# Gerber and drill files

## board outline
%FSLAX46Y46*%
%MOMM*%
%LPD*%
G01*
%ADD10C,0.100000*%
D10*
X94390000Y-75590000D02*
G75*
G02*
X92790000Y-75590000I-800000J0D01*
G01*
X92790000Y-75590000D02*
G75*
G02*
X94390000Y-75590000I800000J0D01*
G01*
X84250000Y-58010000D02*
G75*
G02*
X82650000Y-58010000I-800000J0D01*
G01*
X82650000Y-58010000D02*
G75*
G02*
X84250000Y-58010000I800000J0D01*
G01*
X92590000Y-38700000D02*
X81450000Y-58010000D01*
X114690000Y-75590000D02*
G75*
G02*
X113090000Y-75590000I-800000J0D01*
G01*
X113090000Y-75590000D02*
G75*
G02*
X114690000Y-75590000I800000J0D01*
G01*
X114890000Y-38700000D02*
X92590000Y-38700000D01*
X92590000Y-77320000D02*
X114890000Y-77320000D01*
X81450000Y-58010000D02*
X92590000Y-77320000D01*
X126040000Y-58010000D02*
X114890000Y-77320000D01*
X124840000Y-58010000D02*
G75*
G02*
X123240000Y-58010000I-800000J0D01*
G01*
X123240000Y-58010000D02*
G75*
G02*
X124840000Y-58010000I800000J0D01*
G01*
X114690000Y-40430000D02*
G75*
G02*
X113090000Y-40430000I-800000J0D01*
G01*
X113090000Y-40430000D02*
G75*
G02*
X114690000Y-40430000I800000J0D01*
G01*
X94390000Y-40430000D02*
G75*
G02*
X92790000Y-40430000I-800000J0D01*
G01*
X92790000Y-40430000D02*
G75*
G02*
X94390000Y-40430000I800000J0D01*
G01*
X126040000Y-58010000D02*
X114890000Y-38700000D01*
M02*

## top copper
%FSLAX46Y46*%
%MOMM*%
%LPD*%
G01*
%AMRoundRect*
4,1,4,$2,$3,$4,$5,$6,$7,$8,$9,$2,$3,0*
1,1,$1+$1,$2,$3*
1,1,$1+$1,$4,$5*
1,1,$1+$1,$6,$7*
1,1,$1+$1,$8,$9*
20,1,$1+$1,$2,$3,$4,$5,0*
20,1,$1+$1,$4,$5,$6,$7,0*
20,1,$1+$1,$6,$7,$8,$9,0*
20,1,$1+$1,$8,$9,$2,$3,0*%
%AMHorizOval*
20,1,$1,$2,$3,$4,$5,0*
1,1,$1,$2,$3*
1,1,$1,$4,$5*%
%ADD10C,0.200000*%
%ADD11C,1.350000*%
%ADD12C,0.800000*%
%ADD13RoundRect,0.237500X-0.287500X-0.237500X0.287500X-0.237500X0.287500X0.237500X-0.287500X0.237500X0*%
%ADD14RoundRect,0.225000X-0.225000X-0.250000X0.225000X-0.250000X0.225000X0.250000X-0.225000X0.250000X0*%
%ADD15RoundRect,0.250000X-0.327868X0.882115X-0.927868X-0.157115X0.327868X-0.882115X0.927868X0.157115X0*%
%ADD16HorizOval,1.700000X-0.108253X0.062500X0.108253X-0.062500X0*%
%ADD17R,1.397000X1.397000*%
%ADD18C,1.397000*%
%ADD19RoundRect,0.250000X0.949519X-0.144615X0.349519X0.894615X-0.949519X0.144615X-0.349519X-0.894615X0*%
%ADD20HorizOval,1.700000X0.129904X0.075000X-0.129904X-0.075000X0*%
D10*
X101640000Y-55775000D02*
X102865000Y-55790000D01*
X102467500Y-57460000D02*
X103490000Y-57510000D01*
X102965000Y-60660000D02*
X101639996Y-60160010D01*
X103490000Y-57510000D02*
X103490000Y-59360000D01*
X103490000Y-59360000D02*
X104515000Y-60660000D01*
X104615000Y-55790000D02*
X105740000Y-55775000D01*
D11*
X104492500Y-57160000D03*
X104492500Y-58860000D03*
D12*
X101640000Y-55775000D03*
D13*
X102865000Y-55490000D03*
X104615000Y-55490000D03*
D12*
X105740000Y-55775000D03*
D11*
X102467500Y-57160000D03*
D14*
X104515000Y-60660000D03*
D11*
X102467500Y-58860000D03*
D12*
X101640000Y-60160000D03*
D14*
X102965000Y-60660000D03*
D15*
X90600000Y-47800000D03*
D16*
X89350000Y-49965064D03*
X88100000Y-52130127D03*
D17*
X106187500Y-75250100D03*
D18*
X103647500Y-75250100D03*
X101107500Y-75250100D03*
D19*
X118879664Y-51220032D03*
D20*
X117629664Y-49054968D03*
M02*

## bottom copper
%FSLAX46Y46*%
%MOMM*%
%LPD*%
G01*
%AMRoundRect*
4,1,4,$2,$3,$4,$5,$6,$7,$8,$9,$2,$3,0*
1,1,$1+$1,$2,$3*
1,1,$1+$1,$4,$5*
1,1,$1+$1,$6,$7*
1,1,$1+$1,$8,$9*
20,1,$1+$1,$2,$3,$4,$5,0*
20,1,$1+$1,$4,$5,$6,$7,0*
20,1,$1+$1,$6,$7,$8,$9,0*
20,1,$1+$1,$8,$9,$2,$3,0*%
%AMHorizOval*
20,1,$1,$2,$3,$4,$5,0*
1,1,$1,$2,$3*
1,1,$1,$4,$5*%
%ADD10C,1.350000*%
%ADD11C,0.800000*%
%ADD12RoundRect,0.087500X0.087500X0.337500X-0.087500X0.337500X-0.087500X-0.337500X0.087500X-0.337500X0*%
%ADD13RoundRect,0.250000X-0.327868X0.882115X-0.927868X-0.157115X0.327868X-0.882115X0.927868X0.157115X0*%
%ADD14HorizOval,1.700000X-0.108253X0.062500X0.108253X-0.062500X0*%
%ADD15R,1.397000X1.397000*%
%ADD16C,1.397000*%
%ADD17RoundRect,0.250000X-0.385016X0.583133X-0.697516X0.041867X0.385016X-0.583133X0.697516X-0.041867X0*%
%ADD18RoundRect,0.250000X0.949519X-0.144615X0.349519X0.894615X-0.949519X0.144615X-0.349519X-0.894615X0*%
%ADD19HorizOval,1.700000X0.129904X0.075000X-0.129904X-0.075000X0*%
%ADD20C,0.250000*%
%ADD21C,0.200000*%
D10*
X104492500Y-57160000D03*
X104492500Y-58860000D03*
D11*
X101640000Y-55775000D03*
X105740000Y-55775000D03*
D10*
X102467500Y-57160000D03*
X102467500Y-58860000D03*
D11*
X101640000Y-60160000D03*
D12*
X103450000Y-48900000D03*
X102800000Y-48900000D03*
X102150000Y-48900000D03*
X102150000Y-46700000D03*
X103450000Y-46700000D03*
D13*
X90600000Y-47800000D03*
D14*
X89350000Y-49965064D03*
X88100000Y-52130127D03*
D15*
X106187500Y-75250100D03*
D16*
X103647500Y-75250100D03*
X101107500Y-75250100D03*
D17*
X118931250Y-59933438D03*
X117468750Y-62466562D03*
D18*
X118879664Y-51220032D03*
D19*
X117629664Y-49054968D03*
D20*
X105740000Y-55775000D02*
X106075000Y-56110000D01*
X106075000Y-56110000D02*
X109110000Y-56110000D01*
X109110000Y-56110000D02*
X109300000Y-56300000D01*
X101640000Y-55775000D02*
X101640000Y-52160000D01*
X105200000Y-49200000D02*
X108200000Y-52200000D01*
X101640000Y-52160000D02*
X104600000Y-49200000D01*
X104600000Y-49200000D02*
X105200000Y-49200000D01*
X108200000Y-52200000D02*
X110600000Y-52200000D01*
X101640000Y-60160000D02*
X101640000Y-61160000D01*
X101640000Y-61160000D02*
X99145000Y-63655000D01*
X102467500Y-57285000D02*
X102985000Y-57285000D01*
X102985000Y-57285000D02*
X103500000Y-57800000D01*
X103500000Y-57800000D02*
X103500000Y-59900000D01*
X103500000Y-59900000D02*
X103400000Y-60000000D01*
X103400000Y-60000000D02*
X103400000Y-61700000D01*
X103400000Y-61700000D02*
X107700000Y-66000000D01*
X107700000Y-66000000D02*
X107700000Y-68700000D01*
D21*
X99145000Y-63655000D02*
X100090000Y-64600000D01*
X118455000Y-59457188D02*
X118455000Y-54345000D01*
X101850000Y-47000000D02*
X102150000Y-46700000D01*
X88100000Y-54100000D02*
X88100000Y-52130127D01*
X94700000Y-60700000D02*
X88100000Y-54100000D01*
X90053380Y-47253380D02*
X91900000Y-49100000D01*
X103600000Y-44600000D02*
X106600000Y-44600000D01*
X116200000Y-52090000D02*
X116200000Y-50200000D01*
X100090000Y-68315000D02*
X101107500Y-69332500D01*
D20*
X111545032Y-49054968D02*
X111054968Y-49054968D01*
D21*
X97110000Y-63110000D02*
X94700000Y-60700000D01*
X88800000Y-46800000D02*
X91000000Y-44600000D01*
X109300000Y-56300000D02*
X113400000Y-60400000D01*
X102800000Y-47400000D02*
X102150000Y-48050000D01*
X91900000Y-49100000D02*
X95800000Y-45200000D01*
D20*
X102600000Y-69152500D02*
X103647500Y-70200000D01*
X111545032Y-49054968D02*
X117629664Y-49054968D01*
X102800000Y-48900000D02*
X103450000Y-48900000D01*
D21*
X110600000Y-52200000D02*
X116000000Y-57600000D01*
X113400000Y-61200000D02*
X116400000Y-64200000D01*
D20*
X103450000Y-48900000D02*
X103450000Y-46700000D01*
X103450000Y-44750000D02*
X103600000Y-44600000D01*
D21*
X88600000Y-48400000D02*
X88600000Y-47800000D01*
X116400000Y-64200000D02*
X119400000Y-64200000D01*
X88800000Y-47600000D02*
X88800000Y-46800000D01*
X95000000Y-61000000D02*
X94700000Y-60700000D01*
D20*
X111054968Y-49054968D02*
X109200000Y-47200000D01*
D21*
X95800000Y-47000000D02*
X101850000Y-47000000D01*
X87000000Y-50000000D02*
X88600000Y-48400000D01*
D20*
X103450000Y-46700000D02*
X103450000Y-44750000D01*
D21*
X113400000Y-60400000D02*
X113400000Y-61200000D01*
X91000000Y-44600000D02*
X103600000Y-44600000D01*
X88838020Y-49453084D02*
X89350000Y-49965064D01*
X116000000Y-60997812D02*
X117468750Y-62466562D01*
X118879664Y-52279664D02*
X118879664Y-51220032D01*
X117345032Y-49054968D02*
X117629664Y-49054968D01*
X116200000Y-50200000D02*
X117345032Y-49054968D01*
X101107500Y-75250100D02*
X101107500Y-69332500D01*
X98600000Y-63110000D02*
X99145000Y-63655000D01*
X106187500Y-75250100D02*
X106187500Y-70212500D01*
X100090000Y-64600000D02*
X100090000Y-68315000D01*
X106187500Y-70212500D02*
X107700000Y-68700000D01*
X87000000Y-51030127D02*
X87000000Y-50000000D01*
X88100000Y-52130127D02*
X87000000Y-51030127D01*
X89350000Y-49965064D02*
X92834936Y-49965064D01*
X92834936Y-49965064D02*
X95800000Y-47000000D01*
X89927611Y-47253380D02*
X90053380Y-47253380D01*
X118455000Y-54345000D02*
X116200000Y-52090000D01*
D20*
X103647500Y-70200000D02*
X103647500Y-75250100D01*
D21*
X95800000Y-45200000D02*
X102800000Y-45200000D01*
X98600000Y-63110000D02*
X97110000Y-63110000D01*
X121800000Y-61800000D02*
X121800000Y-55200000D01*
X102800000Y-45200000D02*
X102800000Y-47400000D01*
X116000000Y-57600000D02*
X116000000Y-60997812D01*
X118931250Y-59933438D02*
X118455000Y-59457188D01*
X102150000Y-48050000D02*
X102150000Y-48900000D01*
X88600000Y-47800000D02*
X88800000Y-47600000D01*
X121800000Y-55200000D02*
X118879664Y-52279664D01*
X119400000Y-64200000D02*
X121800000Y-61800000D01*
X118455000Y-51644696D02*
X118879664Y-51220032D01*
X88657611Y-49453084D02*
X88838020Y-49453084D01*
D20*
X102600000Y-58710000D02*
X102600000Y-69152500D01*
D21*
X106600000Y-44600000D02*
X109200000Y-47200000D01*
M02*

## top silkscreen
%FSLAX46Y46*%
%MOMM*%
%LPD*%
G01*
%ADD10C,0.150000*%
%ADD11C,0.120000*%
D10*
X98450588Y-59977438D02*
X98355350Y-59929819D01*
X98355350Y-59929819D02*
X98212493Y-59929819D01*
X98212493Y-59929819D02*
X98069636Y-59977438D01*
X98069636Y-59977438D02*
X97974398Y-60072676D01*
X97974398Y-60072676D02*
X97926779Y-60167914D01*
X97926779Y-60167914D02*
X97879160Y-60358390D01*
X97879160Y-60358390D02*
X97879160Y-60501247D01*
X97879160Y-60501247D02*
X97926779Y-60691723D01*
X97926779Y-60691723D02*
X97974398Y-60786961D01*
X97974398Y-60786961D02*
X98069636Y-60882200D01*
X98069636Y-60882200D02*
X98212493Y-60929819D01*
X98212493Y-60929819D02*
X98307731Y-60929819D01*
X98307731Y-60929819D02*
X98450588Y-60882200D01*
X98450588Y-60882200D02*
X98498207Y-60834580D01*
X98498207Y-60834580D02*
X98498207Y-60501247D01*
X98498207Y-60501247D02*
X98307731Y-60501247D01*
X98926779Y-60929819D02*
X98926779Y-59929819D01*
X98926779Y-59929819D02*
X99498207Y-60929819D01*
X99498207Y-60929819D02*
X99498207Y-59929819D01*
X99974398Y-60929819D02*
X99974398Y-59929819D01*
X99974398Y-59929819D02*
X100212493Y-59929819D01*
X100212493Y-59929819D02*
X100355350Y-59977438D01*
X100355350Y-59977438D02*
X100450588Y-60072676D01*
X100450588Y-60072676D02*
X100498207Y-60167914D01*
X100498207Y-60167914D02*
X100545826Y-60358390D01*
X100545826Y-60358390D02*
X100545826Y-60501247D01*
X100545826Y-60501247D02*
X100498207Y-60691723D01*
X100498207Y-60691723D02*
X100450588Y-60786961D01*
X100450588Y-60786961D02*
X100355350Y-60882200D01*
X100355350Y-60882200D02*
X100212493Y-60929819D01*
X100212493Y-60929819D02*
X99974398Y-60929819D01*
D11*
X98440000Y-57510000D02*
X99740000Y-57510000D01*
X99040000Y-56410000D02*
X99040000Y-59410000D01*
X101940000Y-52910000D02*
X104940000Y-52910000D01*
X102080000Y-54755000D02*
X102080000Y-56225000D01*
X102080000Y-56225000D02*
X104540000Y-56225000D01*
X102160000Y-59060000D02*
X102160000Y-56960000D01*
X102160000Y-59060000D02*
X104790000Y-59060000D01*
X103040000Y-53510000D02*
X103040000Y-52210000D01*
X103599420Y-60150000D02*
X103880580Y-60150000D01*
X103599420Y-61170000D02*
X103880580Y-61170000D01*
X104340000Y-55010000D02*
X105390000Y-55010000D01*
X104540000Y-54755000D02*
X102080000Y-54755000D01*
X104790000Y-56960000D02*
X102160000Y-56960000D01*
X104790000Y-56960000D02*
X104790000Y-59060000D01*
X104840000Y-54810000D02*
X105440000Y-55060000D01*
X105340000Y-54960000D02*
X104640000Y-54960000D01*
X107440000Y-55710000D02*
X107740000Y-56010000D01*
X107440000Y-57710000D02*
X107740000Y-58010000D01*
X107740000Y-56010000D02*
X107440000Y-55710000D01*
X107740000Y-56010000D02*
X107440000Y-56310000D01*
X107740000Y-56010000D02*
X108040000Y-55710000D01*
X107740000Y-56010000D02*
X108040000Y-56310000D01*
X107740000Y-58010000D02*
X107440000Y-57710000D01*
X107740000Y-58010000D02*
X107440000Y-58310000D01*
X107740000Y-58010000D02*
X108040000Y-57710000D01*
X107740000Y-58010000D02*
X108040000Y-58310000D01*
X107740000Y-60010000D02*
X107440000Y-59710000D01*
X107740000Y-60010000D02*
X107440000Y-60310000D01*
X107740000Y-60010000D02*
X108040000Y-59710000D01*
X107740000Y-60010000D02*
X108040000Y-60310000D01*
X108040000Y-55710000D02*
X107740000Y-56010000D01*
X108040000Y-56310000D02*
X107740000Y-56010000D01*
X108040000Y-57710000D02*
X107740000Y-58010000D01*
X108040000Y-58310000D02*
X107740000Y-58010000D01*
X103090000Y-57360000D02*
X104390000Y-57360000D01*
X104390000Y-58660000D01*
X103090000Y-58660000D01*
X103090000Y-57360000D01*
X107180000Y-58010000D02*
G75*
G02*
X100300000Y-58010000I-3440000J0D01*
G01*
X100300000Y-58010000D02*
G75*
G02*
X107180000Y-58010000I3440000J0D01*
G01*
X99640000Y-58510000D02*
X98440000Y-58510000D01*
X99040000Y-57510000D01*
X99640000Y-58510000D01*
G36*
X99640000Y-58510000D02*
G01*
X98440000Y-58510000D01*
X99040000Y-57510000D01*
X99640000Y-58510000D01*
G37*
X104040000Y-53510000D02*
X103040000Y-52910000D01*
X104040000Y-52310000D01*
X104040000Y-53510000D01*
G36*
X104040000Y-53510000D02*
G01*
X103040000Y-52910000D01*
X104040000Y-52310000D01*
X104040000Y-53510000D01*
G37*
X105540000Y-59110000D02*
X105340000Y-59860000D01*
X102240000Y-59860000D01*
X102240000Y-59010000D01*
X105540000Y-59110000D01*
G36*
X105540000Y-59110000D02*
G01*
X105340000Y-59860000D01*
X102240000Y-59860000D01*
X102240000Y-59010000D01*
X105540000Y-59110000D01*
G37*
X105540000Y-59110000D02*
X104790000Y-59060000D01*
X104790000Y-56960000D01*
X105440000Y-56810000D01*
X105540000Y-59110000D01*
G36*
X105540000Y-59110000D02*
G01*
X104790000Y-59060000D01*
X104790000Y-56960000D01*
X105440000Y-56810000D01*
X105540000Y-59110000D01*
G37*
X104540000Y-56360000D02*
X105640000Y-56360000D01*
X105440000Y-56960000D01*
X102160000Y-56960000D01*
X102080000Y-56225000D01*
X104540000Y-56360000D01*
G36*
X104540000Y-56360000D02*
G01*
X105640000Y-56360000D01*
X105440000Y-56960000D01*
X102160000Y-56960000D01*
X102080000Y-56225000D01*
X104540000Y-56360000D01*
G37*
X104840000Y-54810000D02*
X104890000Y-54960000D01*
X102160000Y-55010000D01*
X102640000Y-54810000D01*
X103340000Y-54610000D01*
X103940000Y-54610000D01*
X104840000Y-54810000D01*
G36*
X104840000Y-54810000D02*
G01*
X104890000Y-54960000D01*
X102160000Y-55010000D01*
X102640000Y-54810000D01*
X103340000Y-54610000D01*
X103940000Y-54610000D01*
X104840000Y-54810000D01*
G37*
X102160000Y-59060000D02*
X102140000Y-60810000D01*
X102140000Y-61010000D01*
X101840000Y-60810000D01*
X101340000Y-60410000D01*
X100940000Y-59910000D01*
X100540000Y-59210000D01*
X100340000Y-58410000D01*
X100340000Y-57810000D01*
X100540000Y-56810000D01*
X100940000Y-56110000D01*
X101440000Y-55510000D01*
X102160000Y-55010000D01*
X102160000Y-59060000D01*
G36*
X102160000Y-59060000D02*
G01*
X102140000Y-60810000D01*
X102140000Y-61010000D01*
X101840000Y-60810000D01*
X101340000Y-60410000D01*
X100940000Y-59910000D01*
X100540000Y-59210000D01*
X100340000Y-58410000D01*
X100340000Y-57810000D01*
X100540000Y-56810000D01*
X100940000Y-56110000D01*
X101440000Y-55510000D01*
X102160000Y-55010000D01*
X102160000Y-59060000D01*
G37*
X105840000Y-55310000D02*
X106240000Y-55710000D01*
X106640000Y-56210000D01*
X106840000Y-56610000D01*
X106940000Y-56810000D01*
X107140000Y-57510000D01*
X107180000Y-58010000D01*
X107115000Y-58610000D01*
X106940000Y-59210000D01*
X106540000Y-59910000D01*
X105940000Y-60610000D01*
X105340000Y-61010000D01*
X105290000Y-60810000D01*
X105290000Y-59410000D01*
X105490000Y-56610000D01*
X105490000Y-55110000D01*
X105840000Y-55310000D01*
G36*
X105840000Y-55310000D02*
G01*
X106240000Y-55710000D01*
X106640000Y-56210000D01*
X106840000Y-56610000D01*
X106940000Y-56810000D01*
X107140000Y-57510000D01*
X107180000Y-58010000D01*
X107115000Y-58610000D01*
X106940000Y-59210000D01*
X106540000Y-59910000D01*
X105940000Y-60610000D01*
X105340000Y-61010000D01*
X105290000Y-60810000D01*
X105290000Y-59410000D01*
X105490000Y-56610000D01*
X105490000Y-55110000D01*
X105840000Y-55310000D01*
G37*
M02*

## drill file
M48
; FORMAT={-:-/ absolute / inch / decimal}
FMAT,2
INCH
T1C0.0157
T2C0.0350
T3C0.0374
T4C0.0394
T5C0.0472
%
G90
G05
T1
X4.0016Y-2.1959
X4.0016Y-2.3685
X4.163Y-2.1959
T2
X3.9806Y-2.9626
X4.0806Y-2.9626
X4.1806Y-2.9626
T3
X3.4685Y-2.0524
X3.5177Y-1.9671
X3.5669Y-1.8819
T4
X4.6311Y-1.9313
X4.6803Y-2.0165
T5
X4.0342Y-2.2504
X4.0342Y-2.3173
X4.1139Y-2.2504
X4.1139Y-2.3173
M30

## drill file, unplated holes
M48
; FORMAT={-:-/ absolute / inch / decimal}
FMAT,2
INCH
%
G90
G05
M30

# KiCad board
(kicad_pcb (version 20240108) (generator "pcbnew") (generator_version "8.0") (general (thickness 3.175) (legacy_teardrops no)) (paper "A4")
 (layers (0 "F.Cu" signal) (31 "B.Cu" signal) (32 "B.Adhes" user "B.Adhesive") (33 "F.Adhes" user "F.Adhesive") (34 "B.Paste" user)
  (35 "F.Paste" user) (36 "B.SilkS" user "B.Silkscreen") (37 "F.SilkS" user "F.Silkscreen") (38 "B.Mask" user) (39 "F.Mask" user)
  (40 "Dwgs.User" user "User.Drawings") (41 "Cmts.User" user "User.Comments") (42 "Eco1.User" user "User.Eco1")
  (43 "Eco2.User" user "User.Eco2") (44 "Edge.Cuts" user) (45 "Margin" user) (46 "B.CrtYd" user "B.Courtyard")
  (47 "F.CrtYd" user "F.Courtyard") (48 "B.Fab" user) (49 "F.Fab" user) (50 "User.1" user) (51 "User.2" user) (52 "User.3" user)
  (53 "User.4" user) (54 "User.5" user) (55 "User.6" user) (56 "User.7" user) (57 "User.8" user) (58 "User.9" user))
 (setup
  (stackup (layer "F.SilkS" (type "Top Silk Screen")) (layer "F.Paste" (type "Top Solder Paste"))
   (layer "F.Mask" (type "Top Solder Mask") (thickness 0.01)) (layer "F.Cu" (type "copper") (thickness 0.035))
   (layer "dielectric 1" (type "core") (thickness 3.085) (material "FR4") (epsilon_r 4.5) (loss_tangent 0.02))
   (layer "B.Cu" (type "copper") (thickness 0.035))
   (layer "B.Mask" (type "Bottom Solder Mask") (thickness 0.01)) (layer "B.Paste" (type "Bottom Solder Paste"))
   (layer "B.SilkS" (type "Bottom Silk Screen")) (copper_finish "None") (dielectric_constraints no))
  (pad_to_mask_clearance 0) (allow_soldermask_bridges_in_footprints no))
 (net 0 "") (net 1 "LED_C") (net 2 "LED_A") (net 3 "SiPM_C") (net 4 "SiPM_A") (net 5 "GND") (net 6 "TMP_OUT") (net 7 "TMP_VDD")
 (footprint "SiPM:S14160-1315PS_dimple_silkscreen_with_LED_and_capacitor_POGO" (layer "F.Cu") (at 103.74 58.01)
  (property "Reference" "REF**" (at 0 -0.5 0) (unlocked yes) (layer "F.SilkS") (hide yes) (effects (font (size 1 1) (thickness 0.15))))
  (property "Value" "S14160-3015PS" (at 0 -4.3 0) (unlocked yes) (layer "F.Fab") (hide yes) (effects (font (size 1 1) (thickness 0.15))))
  (fp_line (start -2.1 -2.235) (end -0.875 -2.22) (stroke (width 0.2) (type default)) (layer "F.Cu"))
  (fp_line (start -1.2725 -0.55) (end -0.25 -0.5) (stroke (width 0.2) (type default)) (layer "F.Cu"))
  (fp_line (start -0.775 2.65) (end -2.100004 2.15001) (stroke (width 0.2) (type default)) (layer "F.Cu"))
  (fp_line (start -0.25 -0.5) (end -0.25 1.35) (stroke (width 0.2) (type default)) (layer "F.Cu"))
  (fp_line (start -0.25 1.35) (end 0.775 2.65) (stroke (width 0.2) (type default)) (layer "F.Cu"))
  (fp_line (start 0.875 -2.22) (end 2 -2.235) (stroke (width 0.2) (type default)) (layer "F.Cu"))
  (fp_line (start -5.3 -0.5) (end -4 -0.5) (stroke (width 0.12) (type solid)) (layer "F.SilkS"))
  (fp_line (start -4.7 -1.6) (end -4.7 1.4) (stroke (width 0.12) (type solid)) (layer "F.SilkS"))
  (fp_line (start -1.8 -5.1) (end 1.2 -5.1) (stroke (width 0.12) (type solid)) (layer "F.SilkS"))
  (fp_line (start -1.66 -3.255) (end -1.66 -1.785) (stroke (width 0.12) (type solid)) (layer "F.SilkS"))
  (fp_line (start -1.66 -1.785) (end 0.8 -1.785) (stroke (width 0.12) (type solid)) (layer "F.SilkS"))
  (fp_line (start -1.58 1.05) (end -1.58 -1.05) (stroke (width 0.12) (type solid)) (layer "F.SilkS"))
  (fp_line (start -1.58 1.05) (end 1.05 1.05) (stroke (width 0.12) (type solid)) (layer "F.SilkS"))
  (fp_line (start -0.7 -4.5) (end -0.7 -5.8) (stroke (width 0.12) (type solid)) (layer "F.SilkS"))
  (fp_line (start -0.14058 2.14) (end 0.14058 2.14) (stroke (width 0.12) (type solid)) (layer "F.SilkS"))
  (fp_line (start -0.14058 3.16) (end 0.14058 3.16) (stroke (width 0.12) (type solid)) (layer "F.SilkS"))
  (fp_line (start 0.6 -3) (end 1.65 -3) (stroke (width 0.12) (type default)) (layer "F.SilkS"))
  (fp_line (start 0.8 -3.255) (end -1.66 -3.255) (stroke (width 0.12) (type solid)) (layer "F.SilkS"))
  (fp_line (start 1.05 -1.05) (end -1.58 -1.05) (stroke (width 0.12) (type solid)) (layer "F.SilkS"))
  (fp_line (start 1.05 -1.05) (end 1.05 1.05) (stroke (width 0.12) (type solid)) (layer "F.SilkS"))
  (fp_line (start 1.1 -3.2) (end 1.7 -2.95) (stroke (width 0.12) (type default)) (layer "F.SilkS"))
  (fp_line (start 1.6 -3.05) (end 0.9 -3.05) (stroke (width 0.12) (type default)) (layer "F.SilkS"))
  (fp_line (start 3.7 -2.3) (end 4 -2) (stroke (width 0.12) (type solid)) (layer "F.SilkS"))
  (fp_line (start 3.7 -0.3) (end 4 0) (stroke (width 0.12) (type solid)) (layer "F.SilkS"))
  (fp_line (start 4 -2) (end 3.7 -2.3) (stroke (width 0.12) (type solid)) (layer "F.SilkS"))
  (fp_line (start 4 -2) (end 3.7 -1.7) (stroke (width 0.12) (type solid)) (layer "F.SilkS"))
  (fp_line (start 4 -2) (end 4.3 -2.3) (stroke (width 0.12) (type solid)) (layer "F.SilkS"))
  (fp_line (start 4 -2) (end 4.3 -1.7) (stroke (width 0.12) (type solid)) (layer "F.SilkS"))
  (fp_line (start 4 0) (end 3.7 -0.3) (stroke (width 0.12) (type solid)) (layer "F.SilkS"))
  (fp_line (start 4 0) (end 3.7 0.3) (stroke (width 0.12) (type solid)) (layer "F.SilkS"))
  (fp_line (start 4 0) (end 4.3 -0.3) (stroke (width 0.12) (type solid)) (layer "F.SilkS"))
  (fp_line (start 4 0) (end 4.3 0.3) (stroke (width 0.12) (type solid)) (layer "F.SilkS"))
  (fp_line (start 4 2) (end 3.7 1.7) (stroke (width 0.12) (type solid)) (layer "F.SilkS"))
  (fp_line (start 4 2) (end 3.7 2.3) (stroke (width 0.12) (type solid)) (layer "F.SilkS"))
  (fp_line (start 4 2) (end 4.3 1.7) (stroke (width 0.12) (type solid)) (layer "F.SilkS"))
  (fp_line (start 4 2) (end 4.3 2.3) (stroke (width 0.12) (type solid)) (layer "F.SilkS"))
  (fp_line (start 4.3 -2.3) (end 4 -2) (stroke (width 0.12) (type solid)) (layer "F.SilkS"))
  (fp_line (start 4.3 -1.7) (end 4 -2) (stroke (width 0.12) (type solid)) (layer "F.SilkS"))
  (fp_line (start 4.3 -0.3) (end 4 0) (stroke (width 0.12) (type solid)) (layer "F.SilkS"))
  (fp_line (start 4.3 0.3) (end 4 0) (stroke (width 0.12) (type solid)) (layer "F.SilkS"))
  (fp_rect (start -0.65 -0.65) (end 0.65 0.65) (stroke (width 0.12) (type solid)) (fill none) (layer "F.SilkS"))
  (fp_circle (center 0 0) (end 3.44 0) (stroke (width 0.12) (type solid)) (fill none) (layer "F.SilkS"))
  (fp_poly (pts (xy -4.7 -0.5) (xy -5.3 0.5) (xy -4.1 0.5)) (stroke (width 0.12) (type solid)) (fill solid) (layer "F.SilkS"))
  (fp_poly (pts (xy -0.7 -5.1) (xy 0.3 -4.5) (xy 0.3 -5.7)) (stroke (width 0.12) (type solid)) (fill solid) (layer "F.SilkS"))
  (fp_poly (pts (xy -1.5 1) (xy -1.5 1.85) (xy 1.6 1.85) (xy 1.8 1.1)) (stroke (width 0.12) (type solid)) (fill solid) (layer "F.SilkS"))
  (fp_poly
   (pts (xy 1.05 1.05) (xy 1.8 1.1) (xy 1.7 -1.2) (xy 1.05 -1.05)) (stroke (width 0.12) (type solid)) (fill solid) (layer "F.SilkS"))
  (fp_poly
   (pts (xy 0.8 -1.65) (xy 1.9 -1.65) (xy 1.7 -1.05) (xy -1.58 -1.05) (xy -1.66 -1.785)) (stroke (width 0.12) (type solid)) (fill solid)
   (layer "F.SilkS"))
  (fp_poly
   (pts (xy 1.1 -3.2) (xy 1.15 -3.05) (xy -1.58 -3) (xy -1.1 -3.2) (xy -0.4 -3.4) (xy 0.2 -3.4)) (stroke (width 0.12) (type solid))
   (fill solid) (layer "F.SilkS"))
  (fp_poly
   (pts (xy -1.58 1.05) (xy 1.05 1.05) (xy -1.58 1.05) (xy -1.6 2.8) (xy -1.6 3) (xy -1.9 2.8) (xy -2.4 2.4) (xy -2.8 1.9) (xy -3.2 1.2)
    (xy -3.4 0.4) (xy -3.4 -0.2) (xy -3.2 -1.2) (xy -2.8 -1.9) (xy -2.3 -2.5) (xy -1.58 -3))
   (stroke (width 0.12) (type solid)) (fill solid) (layer "F.SilkS"))
  (fp_poly
   (pts (xy 1.75 -2.9) (xy 2.1 -2.7) (xy 2.5 -2.3) (xy 2.9 -1.8) (xy 3.1 -1.4) (xy 3.2 -1.2) (xy 3.4 -0.5) (xy 3.44 0) (xy 3.375 0.6)
    (xy 3.2 1.2) (xy 2.8 1.9) (xy 2.2 2.6) (xy 1.6 3) (xy 1.55 2.8) (xy 1.55 1.4) (xy 1.75 -1.4))
   (stroke (width 0.12) (type solid)) (fill solid) (layer "F.SilkS"))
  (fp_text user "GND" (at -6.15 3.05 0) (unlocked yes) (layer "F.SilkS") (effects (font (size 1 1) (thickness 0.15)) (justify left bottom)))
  (pad "3" thru_hole circle (at 0.7525 -0.85) (size 1.35 1.35) (drill 1.2) (layers "*.Cu" "*.Mask") (remove_unused_layers no))
  (pad "4" thru_hole circle (at 0.7525 0.85) (size 1.35 1.35) (drill 1.2) (layers "*.Cu" "*.Mask") (remove_unused_layers no))
  (pad "5" thru_hole circle (at -2.1 -2.235) (size 0.8 0.8) (drill 0.4) (layers "*.Cu") (remove_unused_layers no) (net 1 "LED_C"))
  (pad "5" smd roundrect (at -0.875 -2.52) (size 1.05 0.95) (layers "F.Cu" "F.Paste" "F.Mask") (roundrect_rratio 0.25) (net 1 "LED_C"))
  (pad "6" smd roundrect (at 0.875 -2.52) (size 1.05 0.95) (layers "F.Cu" "F.Paste" "F.Mask") (roundrect_rratio 0.25) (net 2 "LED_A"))
  (pad "6" thru_hole circle (at 2 -2.235) (size 0.8 0.8) (drill 0.4) (layers "*.Cu") (remove_unused_layers no) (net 2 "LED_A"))
  (pad "7" thru_hole circle (at -1.2725 -0.85) (size 1.35 1.35) (drill 1.2) (layers "*.Cu" "*.Mask") (remove_unused_layers no)
   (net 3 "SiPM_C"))
  (pad "7" smd roundrect (at 0.775 2.65) (size 0.9 0.95) (layers "F.Cu" "F.Paste" "F.Mask") (roundrect_rratio 0.25) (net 3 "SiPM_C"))
  (pad "8" thru_hole circle (at -1.2725 0.85) (size 1.35 1.35) (drill 1.2) (layers "*.Cu" "*.Mask") (remove_unused_layers no)
   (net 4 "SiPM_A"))
  (pad "9" thru_hole circle (at -2.1 2.15) (size 0.8 0.8) (drill 0.4) (layers "*.Cu") (remove_unused_layers no) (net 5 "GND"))
  (pad "9" smd roundrect (at -0.775 2.65) (size 0.9 0.95) (layers "F.Cu" "F.Paste" "F.Mask") (roundrect_rratio 0.25) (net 5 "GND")))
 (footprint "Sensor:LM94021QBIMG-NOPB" (layer "B.Cu") (at 102.8 47.8 180)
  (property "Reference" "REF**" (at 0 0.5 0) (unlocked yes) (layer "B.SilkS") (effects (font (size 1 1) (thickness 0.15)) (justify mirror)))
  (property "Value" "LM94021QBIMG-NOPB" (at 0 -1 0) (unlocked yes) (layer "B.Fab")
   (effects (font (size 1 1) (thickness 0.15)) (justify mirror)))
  (pad "1" smd roundrect (at -0.65 -1.1 180) (size 0.35 0.85) (layers "B.Cu" "B.Paste" "B.Mask") (roundrect_rratio 0.25) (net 5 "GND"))
  (pad "2" smd roundrect (at 0 -1.1 180) (size 0.35 0.85) (layers "B.Cu" "B.Paste" "B.Mask") (roundrect_rratio 0.25) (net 5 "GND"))
  (pad "3" smd roundrect (at 0.65 -1.1 180) (size 0.35 0.85) (layers "B.Cu" "B.Paste" "B.Mask") (roundrect_rratio 0.25) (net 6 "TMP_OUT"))
  (pad "4" smd roundrect (at 0.65 1.1 180) (size 0.35 0.85) (layers "B.Cu" "B.Paste" "B.Mask") (roundrect_rratio 0.25) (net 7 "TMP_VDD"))
  (pad "5" smd roundrect (at -0.65 1.1 180) (size 0.35 0.85) (layers "B.Cu" "B.Paste" "B.Mask") (roundrect_rratio 0.25) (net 5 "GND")))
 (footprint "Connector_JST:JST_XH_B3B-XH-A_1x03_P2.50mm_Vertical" (layer "B.Cu") (at 90.6 47.8 -120)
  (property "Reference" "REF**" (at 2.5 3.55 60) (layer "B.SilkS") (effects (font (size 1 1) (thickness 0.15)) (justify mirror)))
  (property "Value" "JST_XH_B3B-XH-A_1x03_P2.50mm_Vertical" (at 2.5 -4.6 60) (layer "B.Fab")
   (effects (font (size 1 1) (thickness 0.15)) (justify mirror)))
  (pad "1" thru_hole roundrect (at 0 0 240) (size 1.7 1.95) (drill 0.95) (layers "*.Cu" "*.Mask") (remove_unused_layers no)
   (roundrect_rratio 0.1470588235) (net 6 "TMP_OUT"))
  (pad "2" thru_hole oval (at 2.5 0 240) (size 1.7 1.95) (drill 0.95) (layers "*.Cu" "*.Mask") (remove_unused_layers no) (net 7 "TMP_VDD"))
  (pad "3" thru_hole oval (at 5 0 240) (size 1.7 1.95) (drill 0.95) (layers "*.Cu" "*.Mask") (remove_unused_layers no) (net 5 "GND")))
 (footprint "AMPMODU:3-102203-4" (layer "B.Cu") (at 106.1875 75.2501 180)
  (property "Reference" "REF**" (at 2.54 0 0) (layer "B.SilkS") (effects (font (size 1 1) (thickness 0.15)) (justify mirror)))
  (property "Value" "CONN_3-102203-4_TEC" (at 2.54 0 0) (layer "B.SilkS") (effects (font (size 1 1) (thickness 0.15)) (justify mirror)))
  (pad "1" thru_hole rect (at 0 0 180) (size 1.397 1.397) (drill 0.889) (layers "*.Cu" "*.Mask") (remove_unused_layers no) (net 3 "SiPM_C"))
  (pad "2" thru_hole circle (at 2.54 0 180) (size 1.397 1.397) (drill 0.889) (layers "*.Cu" "*.Mask") (remove_unused_layers no)
   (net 4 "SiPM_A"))
  (pad "3" thru_hole circle (at 5.08 0 180) (size 1.397 1.397) (drill 0.889) (layers "*.Cu" "*.Mask") (remove_unused_layers no)
   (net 5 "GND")))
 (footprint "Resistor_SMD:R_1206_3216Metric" (layer "B.Cu") (at 118.2 61.2 -120)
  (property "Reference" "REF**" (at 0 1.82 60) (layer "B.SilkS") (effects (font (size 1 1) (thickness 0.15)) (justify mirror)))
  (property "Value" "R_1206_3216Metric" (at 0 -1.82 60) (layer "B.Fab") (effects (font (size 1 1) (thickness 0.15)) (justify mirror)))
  (pad "1" smd roundrect (at -1.4625 0 240) (size 1.125 1.75) (layers "B.Cu" "B.Paste" "B.Mask") (roundrect_rratio 0.222222) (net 5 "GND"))
  (pad "2" smd roundrect (at 1.4625 0 240) (size 1.125 1.75) (layers "B.Cu" "B.Paste" "B.Mask") (roundrect_rratio 0.222222) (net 1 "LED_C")))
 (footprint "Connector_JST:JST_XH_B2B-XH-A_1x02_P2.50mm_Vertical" (layer "B.Cu") (at 118.879664 51.220032 120)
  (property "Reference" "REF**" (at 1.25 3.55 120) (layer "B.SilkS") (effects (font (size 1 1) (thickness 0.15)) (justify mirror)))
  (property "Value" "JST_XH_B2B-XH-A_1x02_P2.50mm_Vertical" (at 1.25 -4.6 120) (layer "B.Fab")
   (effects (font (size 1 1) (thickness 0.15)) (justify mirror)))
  (pad "1" thru_hole roundrect (at 0 0 120) (size 1.7 2) (drill 1) (layers "*.Cu" "*.Mask") (remove_unused_layers no)
   (roundrect_rratio 0.1470588235) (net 2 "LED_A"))
  (pad "2" thru_hole oval (at 2.5 0 120) (size 1.7 2) (drill 1) (layers "*.Cu" "*.Mask") (remove_unused_layers no) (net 5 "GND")))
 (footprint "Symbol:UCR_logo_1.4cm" (layer "B.Cu") (at 104.4 43 180)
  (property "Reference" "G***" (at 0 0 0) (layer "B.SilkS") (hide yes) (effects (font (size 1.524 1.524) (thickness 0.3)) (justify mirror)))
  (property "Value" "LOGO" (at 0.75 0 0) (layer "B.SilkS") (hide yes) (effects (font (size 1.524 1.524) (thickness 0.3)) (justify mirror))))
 (gr_circle (center 93.59 75.59) (end 94.39 75.59) (stroke (width 0.1) (type solid)) (fill none) (layer "Edge.Cuts"))
 (gr_circle (center 83.45 58.01) (end 84.25 58.01) (stroke (width 0.1) (type solid)) (fill none) (layer "Edge.Cuts"))
 (gr_line (start 92.59 38.7) (end 81.45 58.01) (stroke (width 0.1) (type solid)) (layer "Edge.Cuts"))
 (gr_circle (center 113.89 75.59) (end 114.69 75.59) (stroke (width 0.1) (type solid)) (fill none) (layer "Edge.Cuts"))
 (gr_line (start 114.89 38.7) (end 92.59 38.7) (stroke (width 0.1) (type solid)) (layer "Edge.Cuts"))
 (gr_line (start 92.59 77.32) (end 114.89 77.32) (stroke (width 0.1) (type solid)) (layer "Edge.Cuts"))
 (gr_line (start 81.45 58.01) (end 92.59 77.32) (stroke (width 0.1) (type solid)) (layer "Edge.Cuts"))
 (gr_line (start 126.04 58.01) (end 114.89 77.32) (stroke (width 0.1) (type solid)) (layer "Edge.Cuts"))
 (gr_circle (center 124.04 58.01) (end 124.84 58.01) (stroke (width 0.1) (type solid)) (fill none) (layer "Edge.Cuts"))
 (gr_circle (center 113.89 40.43) (end 114.69 40.43) (stroke (width 0.1) (type solid)) (fill none) (layer "Edge.Cuts"))
 (gr_circle (center 93.59 40.43) (end 94.39 40.43) (stroke (width 0.1) (type solid)) (fill none) (layer "Edge.Cuts"))
 (gr_line (start 126.04 58.01) (end 114.89 38.7) (stroke (width 0.1) (type solid)) (layer "Edge.Cuts"))
 (segment (start 103.4 61.7) (end 107.7 66) (width 0.25) (layer "B.Cu") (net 3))
 (segment (start 103.4 60) (end 103.4 61.7) (width 0.25) (layer "B.Cu") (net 3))
 (segment (start 102.4675 57.285) (end 102.985 57.285) (width 0.25) (layer "B.Cu") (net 3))
 (segment (start 103.5 59.9) (end 103.4 60) (width 0.25) (layer "B.Cu") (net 3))
 (segment (start 106.1875 75.2501) (end 106.1875 70.2125) (width 0.2) (layer "B.Cu") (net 3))
 (segment (start 102.985 57.285) (end 103.5 57.8) (width 0.25) (layer "B.Cu") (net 3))
 (segment (start 106.1875 70.2125) (end 107.7 68.7) (width 0.2) (layer "B.Cu") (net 3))
 (segment (start 103.5 57.8) (end 103.5 59.9) (width 0.25) (layer "B.Cu") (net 3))
 (segment (start 107.7 66) (end 107.7 68.7) (width 0.25) (layer "B.Cu") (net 3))
 (segment (start 102.6 69.1525) (end 103.6475 70.2) (width 0.25) (layer "B.Cu") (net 4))
 (segment (start 103.6475 70.2) (end 103.6475 75.2501) (width 0.25) (layer "B.Cu") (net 4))
 (segment (start 102.6 58.71) (end 102.6 69.1525) (width 0.25) (layer "B.Cu") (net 4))
 (segment (start 109.3 56.3) (end 113.4 60.4) (width 0.2) (layer "B.Cu") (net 2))
 (segment (start 113.4 61.2) (end 116.4 64.2) (width 0.2) (layer "B.Cu") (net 2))
 (segment (start 116.4 64.2) (end 119.4 64.2) (width 0.2) (layer "B.Cu") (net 2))
 (segment (start 113.4 60.4) (end 113.4 61.2) (width 0.2) (layer "B.Cu") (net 2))
 (segment (start 118.879664 52.279664) (end 118.879664 51.220032) (width 0.2) (layer "B.Cu") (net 2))
 (segment (start 105.74 55.775) (end 106.075 56.11) (width 0.25) (layer "B.Cu") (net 2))
 (segment (start 106.075 56.11) (end 109.11 56.11) (width 0.25) (layer "B.Cu") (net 2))
 (segment (start 109.11 56.11) (end 109.3 56.3) (width 0.25) (layer "B.Cu") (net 2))
 (segment (start 121.8 61.8) (end 121.8 55.2) (width 0.2) (layer "B.Cu") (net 2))
 (segment (start 121.8 55.2) (end 118.879664 52.279664) (width 0.2) (layer "B.Cu") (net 2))
 (segment (start 119.4 64.2) (end 121.8 61.8) (width 0.2) (layer "B.Cu") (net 2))
 (segment (start 118.455 51.644696) (end 118.879664 51.220032) (width 0.2) (layer "B.Cu") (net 2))
 (segment (start 101.64 52.16) (end 104.6 49.2) (width 0.25) (layer "B.Cu") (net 1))
 (segment (start 110.6 52.2) (end 116 57.6) (width 0.2) (layer "B.Cu") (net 1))
 (segment (start 104.6 49.2) (end 105.2 49.2) (width 0.25) (layer "B.Cu") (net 1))
 (segment (start 101.64 55.775) (end 101.64 52.16) (width 0.25) (layer "B.Cu") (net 1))
 (segment (start 105.2 49.2) (end 108.2 52.2) (width 0.25) (layer "B.Cu") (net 1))
 (segment (start 116 60.997812) (end 117.46875 62.466562) (width 0.2) (layer "B.Cu") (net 1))
 (segment (start 108.2 52.2) (end 110.6 52.2) (width 0.25) (layer "B.Cu") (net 1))
 (segment (start 116 57.6) (end 116 60.997812) (width 0.2) (layer "B.Cu") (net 1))
 (segment (start 99.145 63.655) (end 100.09 64.6) (width 0.2) (layer "B.Cu") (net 5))
 (segment (start 118.455 59.457188) (end 118.455 54.345) (width 0.2) (layer "B.Cu") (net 5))
 (segment (start 88.1 54.1) (end 88.1 52.130127) (width 0.2) (layer "B.Cu") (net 5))
 (segment (start 94.7 60.7) (end 88.1 54.1) (width 0.2) (layer "B.Cu") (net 5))
 (segment (start 103.6 44.6) (end 106.6 44.6) (width 0.2) (layer "B.Cu") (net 5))
 (segment (start 116.2 52.09) (end 116.2 50.2) (width 0.2) (layer "B.Cu") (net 5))
 (segment (start 100.09 68.315) (end 101.1075 69.3325) (width 0.2) (layer "B.Cu") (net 5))
 (segment (start 111.545032 49.054968) (end 111.054968 49.054968) (width 0.25) (layer "B.Cu") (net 5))
 (segment (start 97.11 63.11) (end 94.7 60.7) (width 0.2) (layer "B.Cu") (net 5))
 (segment (start 88.8 46.8) (end 91 44.6) (width 0.2) (layer "B.Cu") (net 5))
 (segment (start 111.545032 49.054968) (end 117.629664 49.054968) (width 0.25) (layer "B.Cu") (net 5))
 (segment (start 102.8 48.9) (end 103.45 48.9) (width 0.25) (layer "B.Cu") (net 5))
 (segment (start 103.45 48.9) (end 103.45 46.7) (width 0.25) (layer "B.Cu") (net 5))
 (segment (start 103.45 44.75) (end 103.6 44.6) (width 0.25) (layer "B.Cu") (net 5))
 (segment (start 88.6 48.4) (end 88.6 47.8) (width 0.2) (layer "B.Cu") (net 5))
 (segment (start 88.8 47.6) (end 88.8 46.8) (width 0.2) (layer "B.Cu") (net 5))
 (segment (start 95 61) (end 94.7 60.7) (width 0.2) (layer "B.Cu") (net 5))
 (segment (start 111.054968 49.054968) (end 109.2 47.2) (width 0.25) (layer "B.Cu") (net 5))
 (segment (start 87 50) (end 88.6 48.4) (width 0.2) (layer "B.Cu") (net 5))
 (segment (start 103.45 46.7) (end 103.45 44.75) (width 0.25) (layer "B.Cu") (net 5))
 (segment (start 91 44.6) (end 103.6 44.6) (width 0.2) (layer "B.Cu") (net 5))
 (segment (start 117.345032 49.054968) (end 117.629664 49.054968) (width 0.2) (layer "B.Cu") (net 5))
 (segment (start 101.64 61.16) (end 99.145 63.655) (width 0.25) (layer "B.Cu") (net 5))
 (segment (start 116.2 50.2) (end 117.345032 49.054968) (width 0.2) (layer "B.Cu") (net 5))
 (segment (start 101.1075 75.2501) (end 101.1075 69.3325) (width 0.2) (layer "B.Cu") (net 5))
 (segment (start 98.6 63.11) (end 99.145 63.655) (width 0.2) (layer "B.Cu") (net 5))
 (segment (start 100.09 64.6) (end 100.09 68.315) (width 0.2) (layer "B.Cu") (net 5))
 (segment (start 87 51.030127) (end 87 50) (width 0.2) (layer "B.Cu") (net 5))
 (segment (start 88.1 52.130127) (end 87 51.030127) (width 0.2) (layer "B.Cu") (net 5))
 (segment (start 118.455 54.345) (end 116.2 52.09) (width 0.2) (layer "B.Cu") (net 5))
 (segment (start 98.6 63.11) (end 97.11 63.11) (width 0.2) (layer "B.Cu") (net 5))
 (segment (start 118.93125 59.933438) (end 118.455 59.457188) (width 0.2) (layer "B.Cu") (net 5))
 (segment (start 88.6 47.8) (end 88.8 47.6) (width 0.2) (layer "B.Cu") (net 5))
 (segment (start 101.64 60.16) (end 101.64 61.16) (width 0.25) (layer "B.Cu") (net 5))
 (segment (start 106.6 44.6) (end 109.2 47.2) (width 0.2) (layer "B.Cu") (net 5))
 (segment (start 90.05338 47.25338) (end 91.9 49.1) (width 0.2) (layer "B.Cu") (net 6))
 (segment (start 102.8 47.4) (end 102.15 48.05) (width 0.2) (layer "B.Cu") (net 6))
 (segment (start 91.9 49.1) (end 95.8 45.2) (width 0.2) (layer "B.Cu") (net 6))
 (segment (start 89.927611 47.25338) (end 90.05338 47.25338) (width 0.2) (layer "B.Cu") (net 6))
 (segment (start 95.8 45.2) (end 102.8 45.2) (width 0.2) (layer "B.Cu") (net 6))
 (segment (start 102.8 45.2) (end 102.8 47.4) (width 0.2) (layer "B.Cu") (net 6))
 (segment (start 102.15 48.05) (end 102.15 48.9) (width 0.2) (layer "B.Cu") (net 6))
 (segment (start 101.85 47) (end 102.15 46.7) (width 0.2) (layer "B.Cu") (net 7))
 (segment (start 95.8 47) (end 101.85 47) (width 0.2) (layer "B.Cu") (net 7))
 (segment (start 88.83802 49.453084) (end 89.35 49.965064) (width 0.2) (layer "B.Cu") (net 7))
 (segment (start 89.35 49.965064) (end 92.834936 49.965064) (width 0.2) (layer "B.Cu") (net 7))
 (segment (start 92.834936 49.965064) (end 95.8 47) (width 0.2) (layer "B.Cu") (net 7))
 (segment (start 88.657611 49.453084) (end 88.83802 49.453084) (width 0.2) (layer "B.Cu") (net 7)))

